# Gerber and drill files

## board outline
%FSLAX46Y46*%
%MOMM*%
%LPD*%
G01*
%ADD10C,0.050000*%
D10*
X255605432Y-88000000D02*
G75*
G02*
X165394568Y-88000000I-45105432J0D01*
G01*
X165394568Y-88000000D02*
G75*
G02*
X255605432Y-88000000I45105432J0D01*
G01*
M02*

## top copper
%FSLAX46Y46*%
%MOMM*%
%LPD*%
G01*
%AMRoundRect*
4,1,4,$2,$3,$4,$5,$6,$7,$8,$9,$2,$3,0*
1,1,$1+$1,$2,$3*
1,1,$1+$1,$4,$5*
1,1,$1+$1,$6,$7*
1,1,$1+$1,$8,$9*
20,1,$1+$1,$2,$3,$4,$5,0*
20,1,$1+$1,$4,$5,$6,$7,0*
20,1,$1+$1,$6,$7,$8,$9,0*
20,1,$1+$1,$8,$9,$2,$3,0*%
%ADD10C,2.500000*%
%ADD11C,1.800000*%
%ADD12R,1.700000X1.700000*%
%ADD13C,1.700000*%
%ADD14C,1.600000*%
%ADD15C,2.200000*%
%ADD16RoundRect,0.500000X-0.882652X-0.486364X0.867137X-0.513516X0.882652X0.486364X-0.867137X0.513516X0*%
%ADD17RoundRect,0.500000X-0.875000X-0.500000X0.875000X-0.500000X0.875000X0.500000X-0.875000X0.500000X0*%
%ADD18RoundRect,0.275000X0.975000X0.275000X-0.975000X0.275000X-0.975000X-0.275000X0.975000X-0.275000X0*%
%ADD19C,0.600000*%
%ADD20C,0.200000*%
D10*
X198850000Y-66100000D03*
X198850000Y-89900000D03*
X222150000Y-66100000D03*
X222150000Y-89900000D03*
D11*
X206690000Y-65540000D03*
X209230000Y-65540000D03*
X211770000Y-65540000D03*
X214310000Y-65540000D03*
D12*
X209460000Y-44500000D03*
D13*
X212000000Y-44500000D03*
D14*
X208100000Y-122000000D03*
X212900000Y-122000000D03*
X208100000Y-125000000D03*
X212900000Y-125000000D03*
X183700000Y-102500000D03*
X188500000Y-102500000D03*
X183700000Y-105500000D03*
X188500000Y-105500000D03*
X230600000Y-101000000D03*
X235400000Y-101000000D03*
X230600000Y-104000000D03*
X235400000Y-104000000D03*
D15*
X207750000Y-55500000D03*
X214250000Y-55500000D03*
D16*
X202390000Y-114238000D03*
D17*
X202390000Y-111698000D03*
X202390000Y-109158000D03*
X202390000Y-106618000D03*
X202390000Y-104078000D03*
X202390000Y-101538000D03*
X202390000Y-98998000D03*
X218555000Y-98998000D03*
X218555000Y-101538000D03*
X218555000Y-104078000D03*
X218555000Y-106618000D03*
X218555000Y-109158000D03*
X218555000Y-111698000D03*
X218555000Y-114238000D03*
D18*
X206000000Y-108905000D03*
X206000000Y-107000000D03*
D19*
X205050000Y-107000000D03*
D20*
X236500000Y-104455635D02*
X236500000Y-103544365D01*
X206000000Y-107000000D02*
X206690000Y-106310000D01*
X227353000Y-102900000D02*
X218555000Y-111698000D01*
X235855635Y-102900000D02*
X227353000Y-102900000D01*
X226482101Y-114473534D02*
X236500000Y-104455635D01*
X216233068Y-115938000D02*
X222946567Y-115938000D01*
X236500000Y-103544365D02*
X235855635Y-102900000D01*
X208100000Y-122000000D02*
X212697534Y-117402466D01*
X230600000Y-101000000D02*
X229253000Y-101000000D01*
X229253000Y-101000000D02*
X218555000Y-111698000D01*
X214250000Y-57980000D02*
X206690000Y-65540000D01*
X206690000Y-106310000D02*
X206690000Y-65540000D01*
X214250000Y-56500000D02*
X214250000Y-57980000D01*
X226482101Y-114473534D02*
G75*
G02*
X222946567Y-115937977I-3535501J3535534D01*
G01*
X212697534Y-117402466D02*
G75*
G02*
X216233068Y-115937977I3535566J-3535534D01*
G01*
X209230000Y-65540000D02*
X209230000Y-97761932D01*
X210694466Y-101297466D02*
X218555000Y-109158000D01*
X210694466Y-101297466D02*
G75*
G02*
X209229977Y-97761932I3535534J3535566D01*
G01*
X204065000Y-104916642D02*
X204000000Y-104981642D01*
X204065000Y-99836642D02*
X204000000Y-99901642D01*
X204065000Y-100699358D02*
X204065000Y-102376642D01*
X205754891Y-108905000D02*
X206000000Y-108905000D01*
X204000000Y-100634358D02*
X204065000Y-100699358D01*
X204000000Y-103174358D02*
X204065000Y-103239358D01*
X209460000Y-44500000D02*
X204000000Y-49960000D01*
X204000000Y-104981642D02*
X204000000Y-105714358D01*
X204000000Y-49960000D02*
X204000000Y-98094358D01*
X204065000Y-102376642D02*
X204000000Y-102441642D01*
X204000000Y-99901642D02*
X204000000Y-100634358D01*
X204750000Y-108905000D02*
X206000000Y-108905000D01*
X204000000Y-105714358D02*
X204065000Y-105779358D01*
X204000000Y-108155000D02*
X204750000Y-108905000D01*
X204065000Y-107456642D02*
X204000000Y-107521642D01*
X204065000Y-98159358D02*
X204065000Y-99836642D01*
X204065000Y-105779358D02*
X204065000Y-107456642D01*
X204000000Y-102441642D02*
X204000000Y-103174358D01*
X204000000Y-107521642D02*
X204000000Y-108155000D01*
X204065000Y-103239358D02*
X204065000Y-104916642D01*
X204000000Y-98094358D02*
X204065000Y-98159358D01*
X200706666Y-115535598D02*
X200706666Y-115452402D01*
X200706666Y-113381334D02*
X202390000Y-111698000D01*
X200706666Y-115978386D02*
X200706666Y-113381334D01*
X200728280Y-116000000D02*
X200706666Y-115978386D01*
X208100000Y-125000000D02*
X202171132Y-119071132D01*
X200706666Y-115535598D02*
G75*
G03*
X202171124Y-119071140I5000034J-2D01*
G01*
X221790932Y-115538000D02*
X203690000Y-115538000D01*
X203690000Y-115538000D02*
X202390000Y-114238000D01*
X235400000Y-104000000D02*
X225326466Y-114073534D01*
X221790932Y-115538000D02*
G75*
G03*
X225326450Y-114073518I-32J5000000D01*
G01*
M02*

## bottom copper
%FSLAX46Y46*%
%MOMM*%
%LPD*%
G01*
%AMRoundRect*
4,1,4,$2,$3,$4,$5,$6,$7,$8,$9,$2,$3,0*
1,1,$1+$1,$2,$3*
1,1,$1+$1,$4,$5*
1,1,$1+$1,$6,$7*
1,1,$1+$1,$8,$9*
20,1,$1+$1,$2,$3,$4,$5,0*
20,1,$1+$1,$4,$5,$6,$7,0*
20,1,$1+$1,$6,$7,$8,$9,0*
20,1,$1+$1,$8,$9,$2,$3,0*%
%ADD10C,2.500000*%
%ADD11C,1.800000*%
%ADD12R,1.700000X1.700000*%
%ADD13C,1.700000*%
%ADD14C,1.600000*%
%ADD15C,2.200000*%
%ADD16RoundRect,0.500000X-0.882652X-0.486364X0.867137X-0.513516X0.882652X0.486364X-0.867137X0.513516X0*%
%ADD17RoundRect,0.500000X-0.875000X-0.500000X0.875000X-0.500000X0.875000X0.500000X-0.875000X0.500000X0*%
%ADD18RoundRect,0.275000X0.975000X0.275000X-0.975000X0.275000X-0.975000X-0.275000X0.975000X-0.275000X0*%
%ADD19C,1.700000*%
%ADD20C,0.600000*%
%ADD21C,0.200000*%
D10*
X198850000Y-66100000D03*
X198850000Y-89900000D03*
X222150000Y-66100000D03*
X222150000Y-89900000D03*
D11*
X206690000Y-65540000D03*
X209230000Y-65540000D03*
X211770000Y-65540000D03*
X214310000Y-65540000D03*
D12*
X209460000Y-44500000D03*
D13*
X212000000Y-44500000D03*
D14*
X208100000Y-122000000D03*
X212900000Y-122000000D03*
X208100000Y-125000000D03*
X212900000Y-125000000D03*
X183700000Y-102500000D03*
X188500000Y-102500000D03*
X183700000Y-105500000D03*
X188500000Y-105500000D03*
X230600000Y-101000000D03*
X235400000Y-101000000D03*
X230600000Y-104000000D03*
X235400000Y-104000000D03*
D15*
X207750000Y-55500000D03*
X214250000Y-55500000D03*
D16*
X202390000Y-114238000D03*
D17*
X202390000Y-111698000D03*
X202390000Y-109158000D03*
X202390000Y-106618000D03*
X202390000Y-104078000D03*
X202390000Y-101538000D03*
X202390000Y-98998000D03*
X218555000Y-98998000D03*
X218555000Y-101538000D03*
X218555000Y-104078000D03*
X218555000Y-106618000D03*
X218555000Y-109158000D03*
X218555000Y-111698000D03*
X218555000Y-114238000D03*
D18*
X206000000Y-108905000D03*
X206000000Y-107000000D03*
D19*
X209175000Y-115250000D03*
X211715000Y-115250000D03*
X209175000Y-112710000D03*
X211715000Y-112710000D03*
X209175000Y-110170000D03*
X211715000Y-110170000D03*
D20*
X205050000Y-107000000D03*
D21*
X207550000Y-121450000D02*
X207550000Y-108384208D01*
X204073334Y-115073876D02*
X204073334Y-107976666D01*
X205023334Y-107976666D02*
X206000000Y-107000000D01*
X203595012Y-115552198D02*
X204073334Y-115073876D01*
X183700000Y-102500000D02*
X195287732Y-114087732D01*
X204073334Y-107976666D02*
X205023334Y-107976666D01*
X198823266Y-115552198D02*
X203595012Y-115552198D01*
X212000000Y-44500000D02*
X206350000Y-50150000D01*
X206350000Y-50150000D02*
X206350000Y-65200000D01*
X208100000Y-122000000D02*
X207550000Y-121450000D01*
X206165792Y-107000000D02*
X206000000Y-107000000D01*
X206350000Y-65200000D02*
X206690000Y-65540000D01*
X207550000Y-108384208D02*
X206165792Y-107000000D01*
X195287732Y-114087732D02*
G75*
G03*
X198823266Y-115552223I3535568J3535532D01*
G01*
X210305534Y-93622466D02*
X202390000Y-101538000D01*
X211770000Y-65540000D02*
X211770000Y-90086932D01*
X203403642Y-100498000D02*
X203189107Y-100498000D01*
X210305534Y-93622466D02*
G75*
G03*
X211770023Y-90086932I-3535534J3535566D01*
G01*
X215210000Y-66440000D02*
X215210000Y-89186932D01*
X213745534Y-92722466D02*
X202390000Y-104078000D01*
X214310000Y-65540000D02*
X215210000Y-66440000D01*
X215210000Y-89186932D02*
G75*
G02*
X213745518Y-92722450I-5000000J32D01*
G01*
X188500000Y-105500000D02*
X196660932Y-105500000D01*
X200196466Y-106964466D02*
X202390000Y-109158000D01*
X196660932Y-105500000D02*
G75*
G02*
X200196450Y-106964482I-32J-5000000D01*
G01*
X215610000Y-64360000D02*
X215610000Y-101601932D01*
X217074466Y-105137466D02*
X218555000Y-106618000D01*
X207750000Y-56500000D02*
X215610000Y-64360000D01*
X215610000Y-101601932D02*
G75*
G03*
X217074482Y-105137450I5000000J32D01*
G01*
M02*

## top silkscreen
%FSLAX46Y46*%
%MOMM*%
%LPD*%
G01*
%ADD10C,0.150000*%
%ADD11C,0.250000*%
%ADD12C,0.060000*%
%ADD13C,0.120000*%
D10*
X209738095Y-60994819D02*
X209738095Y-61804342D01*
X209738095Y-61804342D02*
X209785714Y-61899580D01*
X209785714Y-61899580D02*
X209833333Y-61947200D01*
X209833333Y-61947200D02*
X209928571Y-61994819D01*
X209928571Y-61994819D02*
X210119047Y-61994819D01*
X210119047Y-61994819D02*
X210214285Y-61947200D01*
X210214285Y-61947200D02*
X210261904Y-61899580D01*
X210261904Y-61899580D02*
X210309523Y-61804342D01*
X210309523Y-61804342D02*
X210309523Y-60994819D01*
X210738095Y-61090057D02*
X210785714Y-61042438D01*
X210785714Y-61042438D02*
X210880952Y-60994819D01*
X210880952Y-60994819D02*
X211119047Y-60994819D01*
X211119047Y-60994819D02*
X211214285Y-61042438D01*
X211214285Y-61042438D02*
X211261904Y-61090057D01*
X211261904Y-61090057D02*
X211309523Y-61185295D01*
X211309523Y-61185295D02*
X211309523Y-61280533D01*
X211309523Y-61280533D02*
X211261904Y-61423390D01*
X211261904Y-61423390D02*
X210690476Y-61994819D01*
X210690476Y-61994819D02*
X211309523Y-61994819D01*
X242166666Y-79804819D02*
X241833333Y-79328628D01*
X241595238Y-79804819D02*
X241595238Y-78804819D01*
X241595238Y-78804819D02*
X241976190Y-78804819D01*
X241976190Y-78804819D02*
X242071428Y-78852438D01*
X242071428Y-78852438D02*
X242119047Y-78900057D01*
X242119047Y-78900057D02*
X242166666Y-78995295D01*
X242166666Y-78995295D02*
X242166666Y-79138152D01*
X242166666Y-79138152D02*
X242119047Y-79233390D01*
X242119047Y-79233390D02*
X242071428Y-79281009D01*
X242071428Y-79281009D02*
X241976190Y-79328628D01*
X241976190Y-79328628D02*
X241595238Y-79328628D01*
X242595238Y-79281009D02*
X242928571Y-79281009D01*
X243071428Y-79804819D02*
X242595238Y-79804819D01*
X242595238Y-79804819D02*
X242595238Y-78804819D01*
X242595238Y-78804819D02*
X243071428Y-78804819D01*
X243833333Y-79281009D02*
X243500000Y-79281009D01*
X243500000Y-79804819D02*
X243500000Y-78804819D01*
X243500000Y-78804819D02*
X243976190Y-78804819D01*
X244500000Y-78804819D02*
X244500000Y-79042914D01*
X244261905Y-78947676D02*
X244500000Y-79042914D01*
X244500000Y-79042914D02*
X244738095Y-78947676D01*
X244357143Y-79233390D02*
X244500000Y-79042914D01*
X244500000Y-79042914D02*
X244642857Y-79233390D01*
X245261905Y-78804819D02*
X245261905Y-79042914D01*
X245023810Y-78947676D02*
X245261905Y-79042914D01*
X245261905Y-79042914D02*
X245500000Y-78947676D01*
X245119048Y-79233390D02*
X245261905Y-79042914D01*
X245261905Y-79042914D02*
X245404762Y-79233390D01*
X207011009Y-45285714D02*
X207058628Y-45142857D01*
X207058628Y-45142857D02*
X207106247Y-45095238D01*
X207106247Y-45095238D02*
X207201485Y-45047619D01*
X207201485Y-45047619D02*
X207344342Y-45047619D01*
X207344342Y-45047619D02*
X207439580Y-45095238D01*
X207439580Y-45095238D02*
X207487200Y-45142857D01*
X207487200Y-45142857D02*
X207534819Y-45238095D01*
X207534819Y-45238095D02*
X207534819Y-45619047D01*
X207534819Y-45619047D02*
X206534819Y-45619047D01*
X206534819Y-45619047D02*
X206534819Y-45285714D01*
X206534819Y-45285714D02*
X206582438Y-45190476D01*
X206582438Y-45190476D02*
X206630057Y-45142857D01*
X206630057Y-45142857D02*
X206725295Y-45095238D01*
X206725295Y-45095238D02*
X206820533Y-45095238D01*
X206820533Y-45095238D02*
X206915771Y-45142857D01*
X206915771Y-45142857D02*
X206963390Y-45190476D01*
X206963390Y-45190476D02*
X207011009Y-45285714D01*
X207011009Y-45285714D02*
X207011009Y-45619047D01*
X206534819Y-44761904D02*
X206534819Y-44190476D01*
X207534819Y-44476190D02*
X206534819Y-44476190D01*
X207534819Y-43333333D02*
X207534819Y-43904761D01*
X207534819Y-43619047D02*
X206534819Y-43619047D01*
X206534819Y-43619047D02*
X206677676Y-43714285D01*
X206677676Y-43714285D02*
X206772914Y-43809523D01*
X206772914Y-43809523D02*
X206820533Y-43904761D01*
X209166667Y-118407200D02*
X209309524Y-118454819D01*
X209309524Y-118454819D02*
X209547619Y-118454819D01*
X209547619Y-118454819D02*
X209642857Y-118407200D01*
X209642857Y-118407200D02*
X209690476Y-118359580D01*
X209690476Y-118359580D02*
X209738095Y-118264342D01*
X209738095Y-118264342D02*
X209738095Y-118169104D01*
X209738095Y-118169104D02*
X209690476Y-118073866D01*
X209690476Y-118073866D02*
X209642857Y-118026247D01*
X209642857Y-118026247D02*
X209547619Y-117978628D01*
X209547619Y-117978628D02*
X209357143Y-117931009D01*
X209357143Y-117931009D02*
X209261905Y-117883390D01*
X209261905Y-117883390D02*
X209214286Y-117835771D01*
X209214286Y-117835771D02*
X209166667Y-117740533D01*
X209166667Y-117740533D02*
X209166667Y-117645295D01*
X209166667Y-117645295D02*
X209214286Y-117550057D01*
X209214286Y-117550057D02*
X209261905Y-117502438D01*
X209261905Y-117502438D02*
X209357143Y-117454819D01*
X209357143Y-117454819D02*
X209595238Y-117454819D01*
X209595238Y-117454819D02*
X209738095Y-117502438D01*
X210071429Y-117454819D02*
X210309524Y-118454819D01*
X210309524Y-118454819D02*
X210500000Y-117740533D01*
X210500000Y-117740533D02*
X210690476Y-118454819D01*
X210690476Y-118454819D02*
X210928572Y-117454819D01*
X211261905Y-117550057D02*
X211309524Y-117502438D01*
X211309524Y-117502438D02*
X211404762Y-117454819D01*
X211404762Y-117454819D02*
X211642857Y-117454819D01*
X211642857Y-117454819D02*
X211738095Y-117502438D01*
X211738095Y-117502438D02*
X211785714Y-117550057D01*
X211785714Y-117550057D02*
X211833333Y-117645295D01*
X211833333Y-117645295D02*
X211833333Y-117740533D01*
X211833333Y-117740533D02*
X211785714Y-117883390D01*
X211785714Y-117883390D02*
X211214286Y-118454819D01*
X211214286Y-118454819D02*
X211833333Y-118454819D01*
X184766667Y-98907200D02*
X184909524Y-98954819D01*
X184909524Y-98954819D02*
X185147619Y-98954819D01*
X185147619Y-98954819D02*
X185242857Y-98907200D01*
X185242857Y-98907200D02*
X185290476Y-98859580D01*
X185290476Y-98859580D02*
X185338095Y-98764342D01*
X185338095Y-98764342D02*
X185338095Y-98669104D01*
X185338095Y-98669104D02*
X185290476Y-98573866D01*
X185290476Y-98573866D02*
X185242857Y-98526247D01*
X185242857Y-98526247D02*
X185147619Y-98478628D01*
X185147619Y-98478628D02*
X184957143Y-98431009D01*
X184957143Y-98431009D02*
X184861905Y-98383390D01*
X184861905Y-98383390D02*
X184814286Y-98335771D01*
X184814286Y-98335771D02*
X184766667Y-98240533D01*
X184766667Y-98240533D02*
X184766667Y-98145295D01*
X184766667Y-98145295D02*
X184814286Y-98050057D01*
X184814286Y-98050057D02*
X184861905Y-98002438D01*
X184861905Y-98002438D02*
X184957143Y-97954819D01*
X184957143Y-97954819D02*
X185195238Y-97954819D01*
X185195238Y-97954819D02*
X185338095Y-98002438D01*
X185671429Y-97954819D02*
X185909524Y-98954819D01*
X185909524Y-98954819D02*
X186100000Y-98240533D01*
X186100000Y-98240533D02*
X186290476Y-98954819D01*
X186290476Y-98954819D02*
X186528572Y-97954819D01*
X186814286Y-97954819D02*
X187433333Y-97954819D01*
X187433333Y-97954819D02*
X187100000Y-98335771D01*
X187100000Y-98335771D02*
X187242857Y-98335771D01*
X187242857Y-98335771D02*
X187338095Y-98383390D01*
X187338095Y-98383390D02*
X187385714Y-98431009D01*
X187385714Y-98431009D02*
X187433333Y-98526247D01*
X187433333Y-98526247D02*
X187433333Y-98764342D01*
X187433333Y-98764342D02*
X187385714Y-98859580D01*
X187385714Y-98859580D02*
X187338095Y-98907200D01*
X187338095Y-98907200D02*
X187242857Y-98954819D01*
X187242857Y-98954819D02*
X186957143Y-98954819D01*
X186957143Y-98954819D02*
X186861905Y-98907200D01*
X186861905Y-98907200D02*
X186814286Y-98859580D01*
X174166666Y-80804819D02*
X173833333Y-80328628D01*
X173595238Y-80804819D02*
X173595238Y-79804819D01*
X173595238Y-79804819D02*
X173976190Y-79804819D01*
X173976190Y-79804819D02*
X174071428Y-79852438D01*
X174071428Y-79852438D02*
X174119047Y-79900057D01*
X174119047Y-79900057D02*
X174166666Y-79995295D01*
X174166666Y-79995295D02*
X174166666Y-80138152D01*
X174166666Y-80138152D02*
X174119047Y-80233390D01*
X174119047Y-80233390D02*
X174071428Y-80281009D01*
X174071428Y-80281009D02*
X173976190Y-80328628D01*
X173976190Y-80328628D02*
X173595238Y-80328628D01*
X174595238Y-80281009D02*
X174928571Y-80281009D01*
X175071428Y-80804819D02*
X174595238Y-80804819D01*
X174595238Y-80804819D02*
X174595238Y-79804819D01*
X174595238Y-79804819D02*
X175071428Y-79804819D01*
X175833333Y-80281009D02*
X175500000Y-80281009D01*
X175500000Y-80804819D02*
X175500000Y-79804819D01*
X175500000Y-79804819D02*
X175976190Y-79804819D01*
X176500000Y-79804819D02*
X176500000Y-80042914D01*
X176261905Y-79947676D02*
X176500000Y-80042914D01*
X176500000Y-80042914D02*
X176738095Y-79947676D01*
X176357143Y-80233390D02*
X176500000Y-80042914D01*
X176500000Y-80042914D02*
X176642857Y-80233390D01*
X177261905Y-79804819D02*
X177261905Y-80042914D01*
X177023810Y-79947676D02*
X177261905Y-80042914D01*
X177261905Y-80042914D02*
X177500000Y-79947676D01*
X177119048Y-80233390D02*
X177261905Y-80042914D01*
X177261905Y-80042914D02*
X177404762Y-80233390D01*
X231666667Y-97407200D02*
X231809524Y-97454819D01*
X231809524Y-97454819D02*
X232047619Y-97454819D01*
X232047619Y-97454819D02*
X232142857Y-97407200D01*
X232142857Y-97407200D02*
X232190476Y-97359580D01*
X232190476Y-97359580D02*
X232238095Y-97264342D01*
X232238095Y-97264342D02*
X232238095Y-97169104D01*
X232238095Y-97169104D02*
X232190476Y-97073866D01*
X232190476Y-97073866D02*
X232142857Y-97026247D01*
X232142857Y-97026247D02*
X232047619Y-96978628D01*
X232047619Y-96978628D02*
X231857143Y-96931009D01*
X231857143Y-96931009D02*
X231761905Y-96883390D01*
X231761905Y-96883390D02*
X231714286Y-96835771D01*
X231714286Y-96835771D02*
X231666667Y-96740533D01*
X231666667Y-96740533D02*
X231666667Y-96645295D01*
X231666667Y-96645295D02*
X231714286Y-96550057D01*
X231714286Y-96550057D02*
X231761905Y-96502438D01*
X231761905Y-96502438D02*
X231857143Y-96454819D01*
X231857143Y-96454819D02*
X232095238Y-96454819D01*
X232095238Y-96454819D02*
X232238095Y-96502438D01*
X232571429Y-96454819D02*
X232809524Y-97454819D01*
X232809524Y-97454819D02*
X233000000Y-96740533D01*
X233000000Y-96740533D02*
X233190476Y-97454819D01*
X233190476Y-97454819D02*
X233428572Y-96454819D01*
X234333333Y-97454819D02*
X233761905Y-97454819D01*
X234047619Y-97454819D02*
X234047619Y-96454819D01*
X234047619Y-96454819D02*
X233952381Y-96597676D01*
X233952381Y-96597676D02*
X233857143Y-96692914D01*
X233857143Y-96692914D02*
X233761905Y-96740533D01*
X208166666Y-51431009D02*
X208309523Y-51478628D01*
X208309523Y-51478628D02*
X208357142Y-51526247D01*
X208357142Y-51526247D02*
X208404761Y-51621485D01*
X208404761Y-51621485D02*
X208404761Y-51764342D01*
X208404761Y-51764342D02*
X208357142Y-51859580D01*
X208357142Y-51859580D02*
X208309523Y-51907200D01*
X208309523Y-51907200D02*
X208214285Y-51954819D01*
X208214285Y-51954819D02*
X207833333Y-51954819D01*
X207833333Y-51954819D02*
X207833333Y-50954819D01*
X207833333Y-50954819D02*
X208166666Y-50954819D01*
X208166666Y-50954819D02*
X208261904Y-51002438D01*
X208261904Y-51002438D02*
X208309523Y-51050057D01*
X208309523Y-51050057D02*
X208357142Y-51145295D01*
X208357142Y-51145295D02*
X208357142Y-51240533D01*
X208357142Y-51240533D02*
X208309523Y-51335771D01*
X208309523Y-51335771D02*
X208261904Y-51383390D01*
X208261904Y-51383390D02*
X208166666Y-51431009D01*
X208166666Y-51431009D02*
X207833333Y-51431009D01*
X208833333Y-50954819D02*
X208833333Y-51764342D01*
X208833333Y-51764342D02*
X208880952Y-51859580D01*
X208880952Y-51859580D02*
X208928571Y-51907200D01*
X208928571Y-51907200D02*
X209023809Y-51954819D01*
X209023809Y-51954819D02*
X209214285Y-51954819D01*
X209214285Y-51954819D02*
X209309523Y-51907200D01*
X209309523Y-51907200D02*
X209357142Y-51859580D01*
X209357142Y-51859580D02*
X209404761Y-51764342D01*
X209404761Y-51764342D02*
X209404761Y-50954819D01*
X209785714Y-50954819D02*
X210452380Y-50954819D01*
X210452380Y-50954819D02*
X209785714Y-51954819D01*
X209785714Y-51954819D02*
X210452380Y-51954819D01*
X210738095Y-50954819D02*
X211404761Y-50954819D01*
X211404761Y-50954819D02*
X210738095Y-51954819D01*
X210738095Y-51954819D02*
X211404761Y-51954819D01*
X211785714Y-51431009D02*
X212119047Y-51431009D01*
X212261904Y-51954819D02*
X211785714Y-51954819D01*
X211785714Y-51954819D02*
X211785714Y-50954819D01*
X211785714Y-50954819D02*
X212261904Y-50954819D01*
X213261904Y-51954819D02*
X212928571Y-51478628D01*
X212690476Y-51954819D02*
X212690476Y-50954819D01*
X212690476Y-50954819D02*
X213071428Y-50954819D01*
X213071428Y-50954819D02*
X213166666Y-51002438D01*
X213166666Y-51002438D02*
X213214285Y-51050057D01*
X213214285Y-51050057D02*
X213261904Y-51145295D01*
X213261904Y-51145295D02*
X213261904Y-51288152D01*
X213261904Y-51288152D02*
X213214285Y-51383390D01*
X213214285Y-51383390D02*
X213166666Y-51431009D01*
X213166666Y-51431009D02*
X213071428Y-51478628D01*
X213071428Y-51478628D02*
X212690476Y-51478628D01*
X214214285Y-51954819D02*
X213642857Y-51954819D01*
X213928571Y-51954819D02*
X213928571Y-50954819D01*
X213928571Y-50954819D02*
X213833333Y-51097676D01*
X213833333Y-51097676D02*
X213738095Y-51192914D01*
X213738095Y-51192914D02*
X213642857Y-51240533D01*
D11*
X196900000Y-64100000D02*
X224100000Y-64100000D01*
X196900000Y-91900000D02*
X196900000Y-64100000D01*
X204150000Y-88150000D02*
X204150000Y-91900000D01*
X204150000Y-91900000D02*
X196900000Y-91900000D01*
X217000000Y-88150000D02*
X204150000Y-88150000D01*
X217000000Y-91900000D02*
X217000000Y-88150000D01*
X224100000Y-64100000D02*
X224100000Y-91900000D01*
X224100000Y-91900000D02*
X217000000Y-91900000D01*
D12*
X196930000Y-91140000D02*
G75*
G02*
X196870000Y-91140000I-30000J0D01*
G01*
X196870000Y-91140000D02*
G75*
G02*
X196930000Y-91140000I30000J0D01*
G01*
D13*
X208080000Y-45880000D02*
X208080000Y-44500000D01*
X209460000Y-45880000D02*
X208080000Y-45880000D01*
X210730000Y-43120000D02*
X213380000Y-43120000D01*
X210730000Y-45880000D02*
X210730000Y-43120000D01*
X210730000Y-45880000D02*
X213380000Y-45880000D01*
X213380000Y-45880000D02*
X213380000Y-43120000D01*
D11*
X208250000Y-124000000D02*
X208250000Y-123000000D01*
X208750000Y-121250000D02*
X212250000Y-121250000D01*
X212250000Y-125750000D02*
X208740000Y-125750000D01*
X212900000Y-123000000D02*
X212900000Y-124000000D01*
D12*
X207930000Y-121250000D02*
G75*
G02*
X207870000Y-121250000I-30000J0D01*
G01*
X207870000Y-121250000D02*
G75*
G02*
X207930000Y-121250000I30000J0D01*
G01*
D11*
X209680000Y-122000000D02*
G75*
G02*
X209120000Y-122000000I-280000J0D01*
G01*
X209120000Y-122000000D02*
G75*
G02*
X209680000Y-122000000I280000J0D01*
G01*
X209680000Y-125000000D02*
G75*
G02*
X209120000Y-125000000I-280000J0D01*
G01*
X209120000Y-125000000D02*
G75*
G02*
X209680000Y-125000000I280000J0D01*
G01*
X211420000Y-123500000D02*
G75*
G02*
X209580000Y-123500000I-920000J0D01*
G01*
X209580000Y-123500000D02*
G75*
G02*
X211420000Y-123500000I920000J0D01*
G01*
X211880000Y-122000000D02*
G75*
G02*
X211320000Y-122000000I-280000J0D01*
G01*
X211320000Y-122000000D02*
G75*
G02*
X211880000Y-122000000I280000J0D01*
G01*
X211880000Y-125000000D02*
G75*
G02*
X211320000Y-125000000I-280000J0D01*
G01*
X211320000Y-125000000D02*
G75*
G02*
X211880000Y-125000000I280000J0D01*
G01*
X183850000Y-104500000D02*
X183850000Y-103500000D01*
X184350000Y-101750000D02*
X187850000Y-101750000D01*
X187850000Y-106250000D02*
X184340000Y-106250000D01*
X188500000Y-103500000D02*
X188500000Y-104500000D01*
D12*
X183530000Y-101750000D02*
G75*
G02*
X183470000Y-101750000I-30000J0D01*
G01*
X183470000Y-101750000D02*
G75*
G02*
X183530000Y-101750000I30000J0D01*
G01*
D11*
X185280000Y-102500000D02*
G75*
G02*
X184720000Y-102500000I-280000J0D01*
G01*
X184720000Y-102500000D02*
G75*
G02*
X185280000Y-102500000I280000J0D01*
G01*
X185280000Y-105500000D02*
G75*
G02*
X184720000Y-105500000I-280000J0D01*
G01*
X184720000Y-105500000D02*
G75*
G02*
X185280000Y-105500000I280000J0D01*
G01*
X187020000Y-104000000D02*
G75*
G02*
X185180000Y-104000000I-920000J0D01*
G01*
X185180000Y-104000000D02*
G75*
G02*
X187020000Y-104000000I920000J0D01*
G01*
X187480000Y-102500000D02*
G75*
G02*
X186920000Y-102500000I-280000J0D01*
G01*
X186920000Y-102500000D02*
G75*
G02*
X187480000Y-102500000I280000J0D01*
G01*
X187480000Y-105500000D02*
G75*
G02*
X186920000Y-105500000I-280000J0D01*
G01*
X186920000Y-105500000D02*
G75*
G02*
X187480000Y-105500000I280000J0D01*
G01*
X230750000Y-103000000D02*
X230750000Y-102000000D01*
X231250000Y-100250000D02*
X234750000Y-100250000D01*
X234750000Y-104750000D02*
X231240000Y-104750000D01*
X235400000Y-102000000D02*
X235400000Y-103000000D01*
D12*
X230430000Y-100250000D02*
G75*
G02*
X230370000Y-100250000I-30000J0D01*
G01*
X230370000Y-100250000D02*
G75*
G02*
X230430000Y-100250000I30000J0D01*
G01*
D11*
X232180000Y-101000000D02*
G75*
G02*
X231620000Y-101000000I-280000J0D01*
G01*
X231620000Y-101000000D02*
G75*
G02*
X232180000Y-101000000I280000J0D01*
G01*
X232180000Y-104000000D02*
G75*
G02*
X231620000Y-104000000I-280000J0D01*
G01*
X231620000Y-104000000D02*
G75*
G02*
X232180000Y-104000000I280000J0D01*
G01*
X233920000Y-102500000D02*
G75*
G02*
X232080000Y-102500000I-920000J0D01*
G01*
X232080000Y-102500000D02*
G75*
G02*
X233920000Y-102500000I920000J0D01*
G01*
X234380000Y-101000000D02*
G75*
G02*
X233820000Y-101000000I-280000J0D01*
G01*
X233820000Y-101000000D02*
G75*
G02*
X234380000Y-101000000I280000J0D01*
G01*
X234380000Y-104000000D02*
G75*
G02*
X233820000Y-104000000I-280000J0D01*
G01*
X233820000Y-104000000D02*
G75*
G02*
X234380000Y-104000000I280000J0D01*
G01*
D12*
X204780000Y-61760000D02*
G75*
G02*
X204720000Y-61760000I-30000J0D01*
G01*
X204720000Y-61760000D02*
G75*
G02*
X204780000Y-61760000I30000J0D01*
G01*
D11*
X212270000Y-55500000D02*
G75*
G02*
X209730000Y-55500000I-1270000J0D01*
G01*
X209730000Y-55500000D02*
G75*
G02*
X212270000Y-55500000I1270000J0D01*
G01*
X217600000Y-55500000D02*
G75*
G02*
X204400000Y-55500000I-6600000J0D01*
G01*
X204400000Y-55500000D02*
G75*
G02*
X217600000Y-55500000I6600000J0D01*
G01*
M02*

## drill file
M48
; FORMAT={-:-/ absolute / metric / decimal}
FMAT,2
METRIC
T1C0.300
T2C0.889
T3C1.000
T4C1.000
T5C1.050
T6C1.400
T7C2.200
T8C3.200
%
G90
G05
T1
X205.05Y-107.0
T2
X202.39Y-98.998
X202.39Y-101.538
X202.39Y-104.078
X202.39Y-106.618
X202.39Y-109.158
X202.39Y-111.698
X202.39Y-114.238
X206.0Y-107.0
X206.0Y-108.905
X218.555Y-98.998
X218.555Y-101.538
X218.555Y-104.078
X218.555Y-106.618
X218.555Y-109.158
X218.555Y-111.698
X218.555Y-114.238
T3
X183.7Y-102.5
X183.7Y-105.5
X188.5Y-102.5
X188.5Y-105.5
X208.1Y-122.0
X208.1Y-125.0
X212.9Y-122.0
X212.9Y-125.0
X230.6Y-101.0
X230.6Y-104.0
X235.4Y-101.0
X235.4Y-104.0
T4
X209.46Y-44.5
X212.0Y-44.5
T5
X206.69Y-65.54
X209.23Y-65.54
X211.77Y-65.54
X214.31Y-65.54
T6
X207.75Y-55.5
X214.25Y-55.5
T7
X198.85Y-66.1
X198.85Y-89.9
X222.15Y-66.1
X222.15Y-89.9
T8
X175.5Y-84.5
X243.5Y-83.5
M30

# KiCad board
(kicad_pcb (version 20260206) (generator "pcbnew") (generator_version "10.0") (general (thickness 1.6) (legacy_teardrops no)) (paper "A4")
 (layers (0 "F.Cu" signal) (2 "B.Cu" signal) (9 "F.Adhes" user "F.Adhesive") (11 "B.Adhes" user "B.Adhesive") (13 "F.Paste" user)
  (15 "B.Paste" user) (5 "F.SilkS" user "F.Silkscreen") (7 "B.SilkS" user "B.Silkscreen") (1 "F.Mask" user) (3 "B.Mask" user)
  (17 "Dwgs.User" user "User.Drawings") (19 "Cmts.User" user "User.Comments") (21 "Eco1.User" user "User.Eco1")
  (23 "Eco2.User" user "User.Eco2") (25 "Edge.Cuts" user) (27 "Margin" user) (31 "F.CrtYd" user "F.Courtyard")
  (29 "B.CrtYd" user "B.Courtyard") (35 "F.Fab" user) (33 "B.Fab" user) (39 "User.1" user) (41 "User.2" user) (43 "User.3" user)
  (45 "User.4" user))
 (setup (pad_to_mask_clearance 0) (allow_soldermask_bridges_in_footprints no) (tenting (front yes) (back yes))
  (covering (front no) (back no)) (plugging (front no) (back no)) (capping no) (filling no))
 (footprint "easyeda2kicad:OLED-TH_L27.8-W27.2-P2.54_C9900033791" (layer "F.Cu") (at 210.5 65.54)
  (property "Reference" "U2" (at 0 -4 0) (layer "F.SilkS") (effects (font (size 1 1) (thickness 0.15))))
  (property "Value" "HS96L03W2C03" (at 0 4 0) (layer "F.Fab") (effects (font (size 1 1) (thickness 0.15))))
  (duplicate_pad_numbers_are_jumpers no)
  (fp_line (start -13.6 -1.44) (end 13.6 -1.44) (stroke (width 0.25) (type solid)) (layer "F.SilkS"))
  (fp_line (start -13.6 26.36) (end -13.6 -1.44) (stroke (width 0.25) (type solid)) (layer "F.SilkS"))
  (fp_line (start -6.35 22.61) (end -6.35 26.36) (stroke (width 0.25) (type solid)) (layer "F.SilkS"))
  (fp_line (start -6.35 26.36) (end -13.6 26.36) (stroke (width 0.25) (type solid)) (layer "F.SilkS"))
  (fp_line (start 6.5 22.61) (end -6.35 22.61) (stroke (width 0.25) (type solid)) (layer "F.SilkS"))
  (fp_line (start 6.5 26.36) (end 6.5 22.61) (stroke (width 0.25) (type solid)) (layer "F.SilkS"))
  (fp_line (start 13.6 -1.44) (end 13.6 26.36) (stroke (width 0.25) (type solid)) (layer "F.SilkS"))
  (fp_line (start 13.6 26.36) (end 6.5 26.36) (stroke (width 0.25) (type solid)) (layer "F.SilkS"))
  (fp_circle (center -13.6 25.6) (end -13.57 25.6) (stroke (width 0.06) (type solid)) (fill no) (layer "F.SilkS"))
  (pad "" thru_hole circle (at -11.65 0.56) (size 2.5 2.5) (drill 2.2) (layers "*.Cu" "*.Mask") (remove_unused_layers no))
  (pad "" thru_hole circle (at -11.65 24.36) (size 2.5 2.5) (drill 2.2) (layers "*.Cu" "*.Mask") (remove_unused_layers no))
  (pad "" thru_hole circle (at 11.65 0.56) (size 2.5 2.5) (drill 2.2) (layers "*.Cu" "*.Mask") (remove_unused_layers no))
  (pad "" thru_hole circle (at 11.65 24.36) (size 2.5 2.5) (drill 2.2) (layers "*.Cu" "*.Mask") (remove_unused_layers no))
  (pad "1" thru_hole circle (at -3.81 0) (size 1.8 1.8) (drill 1.049986) (layers "*.Cu" "*.Mask") (remove_unused_layers no) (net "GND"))
  (pad "2" thru_hole circle (at -1.27 0) (size 1.8 1.8) (drill 1.049986) (layers "*.Cu" "*.Mask") (remove_unused_layers no) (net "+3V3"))
  (pad "3" thru_hole circle (at 1.27 0) (size 1.8 1.8) (drill 1.049986) (layers "*.Cu" "*.Mask") (remove_unused_layers no)
   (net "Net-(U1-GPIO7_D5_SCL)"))
  (pad "4" thru_hole circle (at 3.81 0) (size 1.8 1.8) (drill 1.049986) (layers "*.Cu" "*.Mask") (remove_unused_layers no)
   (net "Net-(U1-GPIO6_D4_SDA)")))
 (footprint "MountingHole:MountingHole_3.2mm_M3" (layer "F.Cu") (at 243.5 83.5)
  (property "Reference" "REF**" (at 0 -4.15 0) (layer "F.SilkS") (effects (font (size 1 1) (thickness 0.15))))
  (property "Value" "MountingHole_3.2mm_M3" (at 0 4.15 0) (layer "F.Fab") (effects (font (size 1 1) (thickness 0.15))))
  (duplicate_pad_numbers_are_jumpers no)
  (pad "" np_thru_hole circle (at 0 0) (size 3.2 3.2) (drill 3.2) (layers "*.Cu" "*.Mask")))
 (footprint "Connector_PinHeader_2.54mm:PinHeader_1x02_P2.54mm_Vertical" (layer "F.Cu") (at 209.46 44.5 90)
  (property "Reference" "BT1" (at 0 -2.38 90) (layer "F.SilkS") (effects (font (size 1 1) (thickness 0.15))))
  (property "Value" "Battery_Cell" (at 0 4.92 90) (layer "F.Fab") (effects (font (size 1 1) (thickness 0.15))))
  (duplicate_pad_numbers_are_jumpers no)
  (fp_line (start -1.38 -1.38) (end 0 -1.38) (stroke (width 0.12) (type solid)) (layer "F.SilkS"))
  (fp_line (start -1.38 0) (end -1.38 -1.38) (stroke (width 0.12) (type solid)) (layer "F.SilkS"))
  (fp_line (start 1.38 1.27) (end 1.38 3.92) (stroke (width 0.12) (type solid)) (layer "F.SilkS"))
  (fp_line (start -1.38 1.27) (end 1.38 1.27) (stroke (width 0.12) (type solid)) (layer "F.SilkS"))
  (fp_line (start -1.38 1.27) (end -1.38 3.92) (stroke (width 0.12) (type solid)) (layer "F.SilkS"))
  (fp_line (start -1.38 3.92) (end 1.38 3.92) (stroke (width 0.12) (type solid)) (layer "F.SilkS"))
  (pad "1" thru_hole rect (at 0 0 90) (size 1.7 1.7) (drill 1) (layers "*.Cu" "*.Mask") (remove_unused_layers no) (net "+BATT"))
  (pad "2" thru_hole circle (at 0 2.54 90) (size 1.7 1.7) (drill 1) (layers "*.Cu" "*.Mask") (remove_unused_layers no) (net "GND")))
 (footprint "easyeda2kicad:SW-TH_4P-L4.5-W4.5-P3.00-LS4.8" (layer "F.Cu") (at 210.5 123.5)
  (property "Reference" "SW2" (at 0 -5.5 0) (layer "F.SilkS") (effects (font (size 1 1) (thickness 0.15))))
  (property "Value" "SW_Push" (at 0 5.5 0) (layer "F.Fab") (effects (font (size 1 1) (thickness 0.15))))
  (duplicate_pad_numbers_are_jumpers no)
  (fp_line (start -2.25 0.5) (end -2.25 -0.5) (stroke (width 0.25) (type solid)) (layer "F.SilkS"))
  (fp_line (start -1.75 -2.25) (end 1.75 -2.25) (stroke (width 0.25) (type solid)) (layer "F.SilkS"))
  (fp_line (start 1.75 2.25) (end -1.76 2.25) (stroke (width 0.25) (type solid)) (layer "F.SilkS"))
  (fp_line (start 2.4 -0.5) (end 2.4 0.5) (stroke (width 0.25) (type solid)) (layer "F.SilkS"))
  (fp_circle (center -2.6 -2.25) (end -2.57 -2.25) (stroke (width 0.06) (type solid)) (fill no) (layer "F.SilkS"))
  (fp_circle (center -1.1 -1.5) (end -0.82 -1.5) (stroke (width 0.25) (type solid)) (fill no) (layer "F.SilkS"))
  (fp_circle (center -1.1 1.5) (end -0.82 1.5) (stroke (width 0.25) (type solid)) (fill no) (layer "F.SilkS"))
  (fp_circle (center 0 0) (end 0.92 0) (stroke (width 0.25) (type solid)) (fill no) (layer "F.SilkS"))
  (fp_circle (center 1.1 -1.5) (end 1.38 -1.5) (stroke (width 0.25) (type solid)) (fill no) (layer "F.SilkS"))
  (fp_circle (center 1.1 1.5) (end 1.38 1.5) (stroke (width 0.25) (type solid)) (fill no) (layer "F.SilkS"))
  (pad "1" thru_hole circle (at -2.4 -1.5) (size 1.6 1.6) (drill 0.999998) (layers "*.Cu" "*.Mask") (remove_unused_layers no) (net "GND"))
  (pad "1" thru_hole circle (at 2.4 -1.5) (size 1.6 1.6) (drill 0.999998) (layers "*.Cu" "*.Mask") (remove_unused_layers no))
  (pad "2" thru_hole circle (at -2.4 1.5) (size 1.6 1.6) (drill 0.999998) (layers "*.Cu" "*.Mask") (remove_unused_layers no)
   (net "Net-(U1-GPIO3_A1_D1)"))
  (pad "2" thru_hole circle (at 2.4 1.5) (size 1.6 1.6) (drill 0.999998) (layers "*.Cu" "*.Mask") (remove_unused_layers no)))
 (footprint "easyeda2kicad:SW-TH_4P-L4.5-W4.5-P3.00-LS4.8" (layer "F.Cu") (at 186.1 104)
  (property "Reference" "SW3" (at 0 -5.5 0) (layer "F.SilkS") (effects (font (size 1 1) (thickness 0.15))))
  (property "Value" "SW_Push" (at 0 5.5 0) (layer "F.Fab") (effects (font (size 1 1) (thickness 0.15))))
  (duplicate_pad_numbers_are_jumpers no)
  (fp_line (start -2.25 0.5) (end -2.25 -0.5) (stroke (width 0.25) (type solid)) (layer "F.SilkS"))
  (fp_line (start -1.75 -2.25) (end 1.75 -2.25) (stroke (width 0.25) (type solid)) (layer "F.SilkS"))
  (fp_line (start 1.75 2.25) (end -1.76 2.25) (stroke (width 0.25) (type solid)) (layer "F.SilkS"))
  (fp_line (start 2.4 -0.5) (end 2.4 0.5) (stroke (width 0.25) (type solid)) (layer "F.SilkS"))
  (fp_circle (center -2.6 -2.25) (end -2.57 -2.25) (stroke (width 0.06) (type solid)) (fill no) (layer "F.SilkS"))
  (fp_circle (center -1.1 -1.5) (end -0.82 -1.5) (stroke (width 0.25) (type solid)) (fill no) (layer "F.SilkS"))
  (fp_circle (center -1.1 1.5) (end -0.82 1.5) (stroke (width 0.25) (type solid)) (fill no) (layer "F.SilkS"))
  (fp_circle (center 0 0) (end 0.92 0) (stroke (width 0.25) (type solid)) (fill no) (layer "F.SilkS"))
  (fp_circle (center 1.1 -1.5) (end 1.38 -1.5) (stroke (width 0.25) (type solid)) (fill no) (layer "F.SilkS"))
  (fp_circle (center 1.1 1.5) (end 1.38 1.5) (stroke (width 0.25) (type solid)) (fill no) (layer "F.SilkS"))
  (pad "1" thru_hole circle (at -2.4 -1.5) (size 1.6 1.6) (drill 0.999998) (layers "*.Cu" "*.Mask") (remove_unused_layers no) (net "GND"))
  (pad "1" thru_hole circle (at 2.4 -1.5) (size 1.6 1.6) (drill 0.999998) (layers "*.Cu" "*.Mask") (remove_unused_layers no))
  (pad "2" thru_hole circle (at -2.4 1.5) (size 1.6 1.6) (drill 0.999998) (layers "*.Cu" "*.Mask") (remove_unused_layers no))
  (pad "2" thru_hole circle (at 2.4 1.5) (size 1.6 1.6) (drill 0.999998) (layers "*.Cu" "*.Mask") (remove_unused_layers no)
   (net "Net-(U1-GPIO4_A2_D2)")))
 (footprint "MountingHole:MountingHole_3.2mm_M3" (layer "F.Cu") (at 175.5 84.5)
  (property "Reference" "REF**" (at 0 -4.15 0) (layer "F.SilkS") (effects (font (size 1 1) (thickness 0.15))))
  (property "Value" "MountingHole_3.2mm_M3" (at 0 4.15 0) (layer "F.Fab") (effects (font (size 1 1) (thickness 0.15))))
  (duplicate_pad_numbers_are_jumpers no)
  (pad "" np_thru_hole circle (at 0 0) (size 3.2 3.2) (drill 3.2) (layers "*.Cu" "*.Mask")))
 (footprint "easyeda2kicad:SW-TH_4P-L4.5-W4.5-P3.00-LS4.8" (layer "F.Cu") (at 233 102.5)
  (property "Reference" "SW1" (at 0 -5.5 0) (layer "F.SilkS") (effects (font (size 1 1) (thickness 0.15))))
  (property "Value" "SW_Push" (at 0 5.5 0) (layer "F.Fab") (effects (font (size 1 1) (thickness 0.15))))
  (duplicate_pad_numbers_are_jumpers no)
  (fp_line (start -2.25 0.5) (end -2.25 -0.5) (stroke (width 0.25) (type solid)) (layer "F.SilkS"))
  (fp_line (start -1.75 -2.25) (end 1.75 -2.25) (stroke (width 0.25) (type solid)) (layer "F.SilkS"))
  (fp_line (start 1.75 2.25) (end -1.76 2.25) (stroke (width 0.25) (type solid)) (layer "F.SilkS"))
  (fp_line (start 2.4 -0.5) (end 2.4 0.5) (stroke (width 0.25) (type solid)) (layer "F.SilkS"))
  (fp_circle (center -2.6 -2.25) (end -2.57 -2.25) (stroke (width 0.06) (type solid)) (fill no) (layer "F.SilkS"))
  (fp_circle (center -1.1 -1.5) (end -0.82 -1.5) (stroke (width 0.25) (type solid)) (fill no) (layer "F.SilkS"))
  (fp_circle (center -1.1 1.5) (end -0.82 1.5) (stroke (width 0.25) (type solid)) (fill no) (layer "F.SilkS"))
  (fp_circle (center 0 0) (end 0.92 0) (stroke (width 0.25) (type solid)) (fill no) (layer "F.SilkS"))
  (fp_circle (center 1.1 -1.5) (end 1.38 -1.5) (stroke (width 0.25) (type solid)) (fill no) (layer "F.SilkS"))
  (fp_circle (center 1.1 1.5) (end 1.38 1.5) (stroke (width 0.25) (type solid)) (fill no) (layer "F.SilkS"))
  (pad "1" thru_hole circle (at -2.4 -1.5) (size 1.6 1.6) (drill 0.999998) (layers "*.Cu" "*.Mask") (remove_unused_layers no) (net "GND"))
  (pad "1" thru_hole circle (at 2.4 -1.5) (size 1.6 1.6) (drill 0.999998) (layers "*.Cu" "*.Mask") (remove_unused_layers no))
  (pad "2" thru_hole circle (at -2.4 1.5) (size 1.6 1.6) (drill 0.999998) (layers "*.Cu" "*.Mask") (remove_unused_layers no))
  (pad "2" thru_hole circle (at 2.4 1.5) (size 1.6 1.6) (drill 0.999998) (layers "*.Cu" "*.Mask") (remove_unused_layers no)
   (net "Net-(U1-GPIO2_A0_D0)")))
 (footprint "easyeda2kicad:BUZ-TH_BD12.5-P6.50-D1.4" (layer "F.Cu") (at 211 55.5)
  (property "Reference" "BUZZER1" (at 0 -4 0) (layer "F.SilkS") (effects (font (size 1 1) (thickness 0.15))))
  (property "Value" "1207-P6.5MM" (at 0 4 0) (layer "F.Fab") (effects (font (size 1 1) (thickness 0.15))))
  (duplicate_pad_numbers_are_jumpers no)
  (fp_circle (center -6.25 6.26) (end -6.22 6.26) (stroke (width 0.06) (type solid)) (fill no) (layer "F.SilkS"))
  (fp_circle (center 0 0) (end 1.27 0) (stroke (width 0.25) (type solid)) (fill no) (layer "F.SilkS"))
  (fp_circle (center 0 0) (end 6.6 0) (stroke (width 0.25) (type solid)) (fill no) (layer "F.SilkS"))
  (pad "1" thru_hole circle (at -3.25 0) (size 2.2 2.2) (drill 1.399998) (layers "*.Cu" "*.Mask") (remove_unused_layers no)
   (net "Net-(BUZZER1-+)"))
  (pad "2" thru_hole circle (at 3.25 0) (size 2.2 2.2) (drill 1.399998) (layers "*.Cu" "*.Mask") (remove_unused_layers no) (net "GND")))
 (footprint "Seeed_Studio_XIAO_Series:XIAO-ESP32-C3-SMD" (layer "B.Cu") (at 201.555 96.118)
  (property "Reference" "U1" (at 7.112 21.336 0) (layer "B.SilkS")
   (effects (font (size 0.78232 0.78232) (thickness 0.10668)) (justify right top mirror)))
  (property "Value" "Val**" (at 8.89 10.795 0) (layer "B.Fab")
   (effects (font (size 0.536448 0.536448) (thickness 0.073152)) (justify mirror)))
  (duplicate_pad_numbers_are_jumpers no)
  (pad "1" thru_hole roundrect (at 0.835 18.12 359.111) (size 2.75 2) (drill 0.889) (layers "*.Cu" "*.Mask") (remove_unused_layers no)
   (roundrect_rratio 0.25) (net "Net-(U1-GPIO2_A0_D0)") (solder_mask_margin 0.0508) (thermal_bridge_angle 45))
  (pad "2" thru_hole roundrect (at 0.835 15.58) (size 2.75 2) (drill 0.889) (layers "*.Cu" "*.Mask") (remove_unused_layers no)
   (roundrect_rratio 0.25) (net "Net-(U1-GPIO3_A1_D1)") (solder_mask_margin 0.0508) (thermal_bridge_angle 45))
  (pad "3" thru_hole roundrect (at 0.835 13.04) (size 2.75 2) (drill 0.889) (layers "*.Cu" "*.Mask") (remove_unused_layers no)
   (roundrect_rratio 0.25) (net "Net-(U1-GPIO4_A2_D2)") (solder_mask_margin 0.0508) (thermal_bridge_angle 45))
  (pad "4" thru_hole roundrect (at 0.835 10.5) (size 2.75 2) (drill 0.889) (layers "*.Cu" "*.Mask") (remove_unused_layers no)
   (roundrect_rratio 0.25) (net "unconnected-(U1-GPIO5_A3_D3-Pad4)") (solder_mask_margin 0.0508) (thermal_bridge_angle 45))
  (pad "5" thru_hole roundrect (at 0.835 7.96) (size 2.75 2) (drill 0.889) (layers "*.Cu" "*.Mask") (remove_unused_layers no)
   (roundrect_rratio 0.25) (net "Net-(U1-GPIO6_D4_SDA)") (solder_mask_margin 0.0508) (thermal_bridge_angle 45))
  (pad "6" thru_hole roundrect (at 0.835 5.42) (size 2.75 2) (drill 0.889) (layers "*.Cu" "*.Mask") (remove_unused_layers no)
   (roundrect_rratio 0.25) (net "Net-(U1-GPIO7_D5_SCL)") (solder_mask_margin 0.0508) (thermal_bridge_angle 45))
  (pad "7" thru_hole roundrect (at 0.835 2.88) (size 2.75 2) (drill 0.889) (layers "*.Cu" "*.Mask") (remove_unused_layers no)
   (roundrect_rratio 0.25) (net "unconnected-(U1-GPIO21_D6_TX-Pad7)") (solder_mask_margin 0.0508) (thermal_bridge_angle 45))
  (pad "8" thru_hole roundrect (at 17 2.88) (size 2.75 2) (drill 0.889) (layers "*.Cu" "*.Mask") (remove_unused_layers no)
   (roundrect_rratio 0.25) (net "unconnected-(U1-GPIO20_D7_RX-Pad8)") (solder_mask_margin 0.0508) (thermal_bridge_angle 45))
  (pad "9" thru_hole roundrect (at 17 5.42) (size 2.75 2) (drill 0.889) (layers "*.Cu" "*.Mask") (remove_unused_layers no)
   (roundrect_rratio 0.25) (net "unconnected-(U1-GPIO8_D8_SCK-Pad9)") (solder_mask_margin 0.0508) (thermal_bridge_angle 45))
  (pad "10" thru_hole roundrect (at 17 7.96) (size 2.75 2) (drill 0.889) (layers "*.Cu" "*.Mask") (remove_unused_layers no)
   (roundrect_rratio 0.25) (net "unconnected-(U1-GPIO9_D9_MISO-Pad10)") (solder_mask_margin 0.0508) (thermal_bridge_angle 45))
  (pad "11" thru_hole roundrect (at 17 10.5) (size 2.75 2) (drill 0.889) (layers "*.Cu" "*.Mask") (remove_unused_layers no)
   (roundrect_rratio 0.25) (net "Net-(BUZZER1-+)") (solder_mask_margin 0.0508) (thermal_bridge_angle 45))
  (pad "12" thru_hole roundrect (at 17 13.04) (size 2.75 2) (drill 0.889) (layers "*.Cu" "*.Mask") (remove_unused_layers no)
   (roundrect_rratio 0.25) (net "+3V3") (solder_mask_margin 0.0508) (thermal_bridge_angle 45))
  (pad "13" thru_hole roundrect (at 17 15.58) (size 2.75 2) (drill 0.889) (layers "*.Cu" "*.Mask") (remove_unused_layers no)
   (roundrect_rratio 0.25) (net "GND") (solder_mask_margin 0.0508) (thermal_bridge_angle 45))
  (pad "14" thru_hole roundrect (at 17 18.12) (size 2.75 2) (drill 0.889) (layers "*.Cu" "*.Mask") (remove_unused_layers no)
   (roundrect_rratio 0.25) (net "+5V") (solder_mask_margin 0.0508) (thermal_bridge_angle 45))
  (pad "15" thru_hole roundrect (at 4.445 12.787 180) (size 2.5 1.1) (drill 0.889) (layers "*.Cu" "*.Mask") (remove_unused_layers no)
   (roundrect_rratio 0.25) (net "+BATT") (thermal_bridge_angle 45))
  (pad "16" thru_hole roundrect (at 4.445 10.882 180) (size 2.5 1.1) (drill 0.889) (layers "*.Cu" "*.Mask") (remove_unused_layers no)
   (roundrect_rratio 0.25) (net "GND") (thermal_bridge_angle 45))
  (pad "17" smd circle (at 7.62 19.132) (size 1.7 1.7) (layers "B.Cu" "B.Mask" "B.Paste") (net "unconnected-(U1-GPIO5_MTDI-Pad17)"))
  (pad "18" smd circle (at 10.16 19.132) (size 1.7 1.7) (layers "B.Cu" "B.Mask" "B.Paste") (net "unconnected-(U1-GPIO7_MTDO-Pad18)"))
  (pad "19" smd circle (at 7.62 16.592) (size 1.7 1.7) (layers "B.Cu" "B.Mask" "B.Paste") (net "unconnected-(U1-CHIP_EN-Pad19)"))
  (pad "20" smd circle (at 10.16 16.592) (size 1.7 1.7) (layers "B.Cu" "B.Mask" "B.Paste") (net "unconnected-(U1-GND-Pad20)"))
  (pad "21" smd circle (at 7.62 14.052) (size 1.7 1.7) (layers "B.Cu" "B.Mask" "B.Paste") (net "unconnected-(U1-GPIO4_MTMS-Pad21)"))
  (pad "22" smd circle (at 10.16 14.052) (size 1.7 1.7) (layers "B.Cu" "B.Mask" "B.Paste") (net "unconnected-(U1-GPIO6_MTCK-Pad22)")))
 (gr_circle (center 210.5 88) (end 247 61.5) (stroke (width 0.05) (type default)) (fill no) (layer "Edge.Cuts"))
 (segment (start 236.5 104.455635) (end 236.5 103.544365) (width 0.2) (layer "F.Cu") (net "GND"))
 (segment (start 206 107) (end 206.69 106.31) (width 0.2) (layer "F.Cu") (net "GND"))
 (segment (start 227.353 102.9) (end 218.555 111.698) (width 0.2) (layer "F.Cu") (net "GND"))
 (segment (start 235.855635 102.9) (end 227.353 102.9) (width 0.2) (layer "F.Cu") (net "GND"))
 (segment (start 226.482101 114.473534) (end 236.5 104.455635) (width 0.2) (layer "F.Cu") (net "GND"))
 (segment (start 216.233068 115.938) (end 222.946567 115.938) (width 0.2) (layer "F.Cu") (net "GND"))
 (segment (start 236.5 103.544365) (end 235.855635 102.9) (width 0.2) (layer "F.Cu") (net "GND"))
 (segment (start 208.1 122) (end 212.697534 117.402466) (width 0.2) (layer "F.Cu") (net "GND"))
 (segment (start 230.6 101) (end 229.253 101) (width 0.2) (layer "F.Cu") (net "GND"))
 (segment (start 229.253 101) (end 218.555 111.698) (width 0.2) (layer "F.Cu") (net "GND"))
 (segment (start 214.25 57.98) (end 206.69 65.54) (width 0.2) (layer "F.Cu") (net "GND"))
 (segment (start 206.69 106.31) (end 206.69 65.54) (width 0.2) (layer "F.Cu") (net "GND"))
 (segment (start 214.25 56.5) (end 214.25 57.98) (width 0.2) (layer "F.Cu") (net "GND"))
 (via (at 205.05 107) (size 0.6) (drill 0.3) (layers "F.Cu" "B.Cu") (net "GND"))
 (arc (start 226.482101 114.473534) (mid 224.859984 115.557398) (end 222.946567 115.938) (width 0.2) (layer "F.Cu") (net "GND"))
 (arc (start 212.697534 117.402466) (mid 214.319651 116.318602) (end 216.233068 115.938) (width 0.2) (layer "F.Cu") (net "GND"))
 (segment (start 207.55 121.45) (end 207.55 108.384208) (width 0.2) (layer "B.Cu") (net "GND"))
 (segment (start 204.073334 115.073876) (end 204.073334 107.976666) (width 0.2) (layer "B.Cu") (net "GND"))
 (segment (start 205.023334 107.976666) (end 206 107) (width 0.2) (layer "B.Cu") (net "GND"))
 (segment (start 203.595012 115.552198) (end 204.073334 115.073876) (width 0.2) (layer "B.Cu") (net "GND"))
 (segment (start 183.7 102.5) (end 195.287732 114.087732) (width 0.2) (layer "B.Cu") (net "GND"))
 (segment (start 204.073334 107.976666) (end 205.023334 107.976666) (width 0.2) (layer "B.Cu") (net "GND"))
 (segment (start 198.823266 115.552198) (end 203.595012 115.552198) (width 0.2) (layer "B.Cu") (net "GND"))
 (segment (start 212 44.5) (end 206.35 50.15) (width 0.2) (layer "B.Cu") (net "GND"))
 (segment (start 206.35 50.15) (end 206.35 65.2) (width 0.2) (layer "B.Cu") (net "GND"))
 (segment (start 208.1 122) (end 207.55 121.45) (width 0.2) (layer "B.Cu") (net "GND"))
 (segment (start 206.165792 107) (end 206 107) (width 0.2) (layer "B.Cu") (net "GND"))
 (segment (start 206.35 65.2) (end 206.69 65.54) (width 0.2) (layer "B.Cu") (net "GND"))
 (segment (start 207.55 108.384208) (end 206.165792 107) (width 0.2) (layer "B.Cu") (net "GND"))
 (arc (start 195.287732 114.087732) (mid 196.909849 115.171596) (end 198.823266 115.552198) (width 0.2) (layer "B.Cu") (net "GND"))
 (segment (start 209.23 65.54) (end 209.23 97.761932) (width 0.2) (layer "F.Cu") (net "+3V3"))
 (segment (start 210.694466 101.297466) (end 218.555 109.158) (width 0.2) (layer "F.Cu") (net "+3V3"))
 (arc (start 210.694466 101.297466) (mid 209.610602 99.675349) (end 209.23 97.761932) (width 0.2) (layer "F.Cu") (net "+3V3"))
 (segment (start 210.305534 93.622466) (end 202.39 101.538) (width 0.2) (layer "B.Cu") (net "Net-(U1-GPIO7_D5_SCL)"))
 (segment (start 211.77 65.54) (end 211.77 90.086932) (width 0.2) (layer "B.Cu") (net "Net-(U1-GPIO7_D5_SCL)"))
 (segment (start 203.403642 100.498) (end 203.189107 100.498) (width 0.2) (layer "B.Cu") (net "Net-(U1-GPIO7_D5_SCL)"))
 (arc (start 210.305534 93.622466) (mid 211.389398 92.000349) (end 211.77 90.086932) (width 0.2) (layer "B.Cu")
  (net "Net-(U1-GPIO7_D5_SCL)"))
 (segment (start 215.21 66.44) (end 215.21 89.186932) (width 0.2) (layer "B.Cu") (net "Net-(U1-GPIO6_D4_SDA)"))
 (segment (start 213.745534 92.722466) (end 202.39 104.078) (width 0.2) (layer "B.Cu") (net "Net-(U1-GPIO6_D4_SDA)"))
 (segment (start 214.31 65.54) (end 215.21 66.44) (width 0.2) (layer "B.Cu") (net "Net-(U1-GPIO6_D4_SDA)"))
 (arc (start 215.21 89.186932) (mid 214.829398 91.100349) (end 213.745534 92.722466) (width 0.2) (layer "B.Cu")
  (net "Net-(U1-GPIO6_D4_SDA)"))
 (segment (start 204.065 104.916642) (end 204 104.981642) (width 0.2) (layer "F.Cu") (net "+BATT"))
 (segment (start 204.065 99.836642) (end 204 99.901642) (width 0.2) (layer "F.Cu") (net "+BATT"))
 (segment (start 204.065 100.699358) (end 204.065 102.376642) (width 0.2) (layer "F.Cu") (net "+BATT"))
 (segment (start 205.754891 108.905) (end 206 108.905) (width 0.2) (layer "F.Cu") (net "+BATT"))
 (segment (start 204 100.634358) (end 204.065 100.699358) (width 0.2) (layer "F.Cu") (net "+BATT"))
 (segment (start 204 103.174358) (end 204.065 103.239358) (width 0.2) (layer "F.Cu") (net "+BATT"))
 (segment (start 209.46 44.5) (end 204 49.96) (width 0.2) (layer "F.Cu") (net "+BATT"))
 (segment (start 204 104.981642) (end 204 105.714358) (width 0.2) (layer "F.Cu") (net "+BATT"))
 (segment (start 204 49.96) (end 204 98.094358) (width 0.2) (layer "F.Cu") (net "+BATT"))
 (segment (start 204.065 102.376642) (end 204 102.441642) (width 0.2) (layer "F.Cu") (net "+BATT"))
 (segment (start 204 99.901642) (end 204 100.634358) (width 0.2) (layer "F.Cu") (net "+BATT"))
 (segment (start 204.75 108.905) (end 206 108.905) (width 0.2) (layer "F.Cu") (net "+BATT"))
 (segment (start 204 105.714358) (end 204.065 105.779358) (width 0.2) (layer "F.Cu") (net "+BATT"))
 (segment (start 204 108.155) (end 204.75 108.905) (width 0.2) (layer "F.Cu") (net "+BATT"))
 (segment (start 204.065 107.456642) (end 204 107.521642) (width 0.2) (layer "F.Cu") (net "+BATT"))
 (segment (start 204.065 98.159358) (end 204.065 99.836642) (width 0.2) (layer "F.Cu") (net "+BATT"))
 (segment (start 204.065 105.779358) (end 204.065 107.456642) (width 0.2) (layer "F.Cu") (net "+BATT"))
 (segment (start 204 102.441642) (end 204 103.174358) (width 0.2) (layer "F.Cu") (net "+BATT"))
 (segment (start 204 107.521642) (end 204 108.155) (width 0.2) (layer "F.Cu") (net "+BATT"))
 (segment (start 204.065 103.239358) (end 204.065 104.916642) (width 0.2) (layer "F.Cu") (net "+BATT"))
 (segment (start 204 98.094358) (end 204.065 98.159358) (width 0.2) (layer "F.Cu") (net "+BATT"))
 (segment (start 200.706666 115.535598) (end 200.706666 115.452402) (width 0.2) (layer "F.Cu") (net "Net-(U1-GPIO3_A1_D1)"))
 (segment (start 200.706666 113.381334) (end 202.39 111.698) (width 0.2) (layer "F.Cu") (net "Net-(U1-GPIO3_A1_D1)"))
 (segment (start 200.706666 115.978386) (end 200.706666 113.381334) (width 0.2) (layer "F.Cu") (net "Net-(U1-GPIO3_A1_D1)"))
 (segment (start 200.72828 116) (end 200.706666 115.978386) (width 0.2) (layer "F.Cu") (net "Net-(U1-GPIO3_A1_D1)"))
 (segment (start 208.1 125) (end 202.171132 119.071132) (width 0.2) (layer "F.Cu") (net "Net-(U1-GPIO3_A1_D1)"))
 (arc (start 200.706666 115.535598) (mid 201.087268 117.449015) (end 202.171132 119.071132) (width 0.2) (layer "F.Cu")
  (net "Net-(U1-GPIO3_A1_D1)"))
 (segment (start 188.5 105.5) (end 196.660932 105.5) (width 0.2) (layer "B.Cu") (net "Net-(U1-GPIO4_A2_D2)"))
 (segment (start 200.196466 106.964466) (end 202.39 109.158) (width 0.2) (layer "B.Cu") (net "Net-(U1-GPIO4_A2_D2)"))
 (arc (start 196.660932 105.5) (mid 198.574349 105.880602) (end 200.196466 106.964466) (width 0.2) (layer "B.Cu")
  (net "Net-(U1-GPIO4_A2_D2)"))
 (segment (start 221.790932 115.538) (end 203.69 115.538) (width 0.2) (layer "F.Cu") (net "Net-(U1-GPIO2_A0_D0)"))
 (segment (start 203.69 115.538) (end 202.39 114.238) (width 0.2) (layer "F.Cu") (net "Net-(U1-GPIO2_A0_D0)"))
 (segment (start 235.4 104) (end 225.326466 114.073534) (width 0.2) (layer "F.Cu") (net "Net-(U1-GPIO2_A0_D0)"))
 (arc (start 221.790932 115.538) (mid 223.704349 115.157398) (end 225.326466 114.073534) (width 0.2) (layer "F.Cu")
  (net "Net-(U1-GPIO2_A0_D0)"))
 (segment (start 215.61 64.36) (end 215.61 101.601932) (width 0.2) (layer "B.Cu") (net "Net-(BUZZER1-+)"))
 (segment (start 217.074466 105.137466) (end 218.555 106.618) (width 0.2) (layer "B.Cu") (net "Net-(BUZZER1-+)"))
 (segment (start 207.75 56.5) (end 215.61 64.36) (width 0.2) (layer "B.Cu") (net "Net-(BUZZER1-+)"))
 (arc (start 215.61 101.601932) (mid 215.990602 103.515349) (end 217.074466 105.137466) (width 0.2) (layer "B.Cu") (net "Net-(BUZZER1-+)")))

